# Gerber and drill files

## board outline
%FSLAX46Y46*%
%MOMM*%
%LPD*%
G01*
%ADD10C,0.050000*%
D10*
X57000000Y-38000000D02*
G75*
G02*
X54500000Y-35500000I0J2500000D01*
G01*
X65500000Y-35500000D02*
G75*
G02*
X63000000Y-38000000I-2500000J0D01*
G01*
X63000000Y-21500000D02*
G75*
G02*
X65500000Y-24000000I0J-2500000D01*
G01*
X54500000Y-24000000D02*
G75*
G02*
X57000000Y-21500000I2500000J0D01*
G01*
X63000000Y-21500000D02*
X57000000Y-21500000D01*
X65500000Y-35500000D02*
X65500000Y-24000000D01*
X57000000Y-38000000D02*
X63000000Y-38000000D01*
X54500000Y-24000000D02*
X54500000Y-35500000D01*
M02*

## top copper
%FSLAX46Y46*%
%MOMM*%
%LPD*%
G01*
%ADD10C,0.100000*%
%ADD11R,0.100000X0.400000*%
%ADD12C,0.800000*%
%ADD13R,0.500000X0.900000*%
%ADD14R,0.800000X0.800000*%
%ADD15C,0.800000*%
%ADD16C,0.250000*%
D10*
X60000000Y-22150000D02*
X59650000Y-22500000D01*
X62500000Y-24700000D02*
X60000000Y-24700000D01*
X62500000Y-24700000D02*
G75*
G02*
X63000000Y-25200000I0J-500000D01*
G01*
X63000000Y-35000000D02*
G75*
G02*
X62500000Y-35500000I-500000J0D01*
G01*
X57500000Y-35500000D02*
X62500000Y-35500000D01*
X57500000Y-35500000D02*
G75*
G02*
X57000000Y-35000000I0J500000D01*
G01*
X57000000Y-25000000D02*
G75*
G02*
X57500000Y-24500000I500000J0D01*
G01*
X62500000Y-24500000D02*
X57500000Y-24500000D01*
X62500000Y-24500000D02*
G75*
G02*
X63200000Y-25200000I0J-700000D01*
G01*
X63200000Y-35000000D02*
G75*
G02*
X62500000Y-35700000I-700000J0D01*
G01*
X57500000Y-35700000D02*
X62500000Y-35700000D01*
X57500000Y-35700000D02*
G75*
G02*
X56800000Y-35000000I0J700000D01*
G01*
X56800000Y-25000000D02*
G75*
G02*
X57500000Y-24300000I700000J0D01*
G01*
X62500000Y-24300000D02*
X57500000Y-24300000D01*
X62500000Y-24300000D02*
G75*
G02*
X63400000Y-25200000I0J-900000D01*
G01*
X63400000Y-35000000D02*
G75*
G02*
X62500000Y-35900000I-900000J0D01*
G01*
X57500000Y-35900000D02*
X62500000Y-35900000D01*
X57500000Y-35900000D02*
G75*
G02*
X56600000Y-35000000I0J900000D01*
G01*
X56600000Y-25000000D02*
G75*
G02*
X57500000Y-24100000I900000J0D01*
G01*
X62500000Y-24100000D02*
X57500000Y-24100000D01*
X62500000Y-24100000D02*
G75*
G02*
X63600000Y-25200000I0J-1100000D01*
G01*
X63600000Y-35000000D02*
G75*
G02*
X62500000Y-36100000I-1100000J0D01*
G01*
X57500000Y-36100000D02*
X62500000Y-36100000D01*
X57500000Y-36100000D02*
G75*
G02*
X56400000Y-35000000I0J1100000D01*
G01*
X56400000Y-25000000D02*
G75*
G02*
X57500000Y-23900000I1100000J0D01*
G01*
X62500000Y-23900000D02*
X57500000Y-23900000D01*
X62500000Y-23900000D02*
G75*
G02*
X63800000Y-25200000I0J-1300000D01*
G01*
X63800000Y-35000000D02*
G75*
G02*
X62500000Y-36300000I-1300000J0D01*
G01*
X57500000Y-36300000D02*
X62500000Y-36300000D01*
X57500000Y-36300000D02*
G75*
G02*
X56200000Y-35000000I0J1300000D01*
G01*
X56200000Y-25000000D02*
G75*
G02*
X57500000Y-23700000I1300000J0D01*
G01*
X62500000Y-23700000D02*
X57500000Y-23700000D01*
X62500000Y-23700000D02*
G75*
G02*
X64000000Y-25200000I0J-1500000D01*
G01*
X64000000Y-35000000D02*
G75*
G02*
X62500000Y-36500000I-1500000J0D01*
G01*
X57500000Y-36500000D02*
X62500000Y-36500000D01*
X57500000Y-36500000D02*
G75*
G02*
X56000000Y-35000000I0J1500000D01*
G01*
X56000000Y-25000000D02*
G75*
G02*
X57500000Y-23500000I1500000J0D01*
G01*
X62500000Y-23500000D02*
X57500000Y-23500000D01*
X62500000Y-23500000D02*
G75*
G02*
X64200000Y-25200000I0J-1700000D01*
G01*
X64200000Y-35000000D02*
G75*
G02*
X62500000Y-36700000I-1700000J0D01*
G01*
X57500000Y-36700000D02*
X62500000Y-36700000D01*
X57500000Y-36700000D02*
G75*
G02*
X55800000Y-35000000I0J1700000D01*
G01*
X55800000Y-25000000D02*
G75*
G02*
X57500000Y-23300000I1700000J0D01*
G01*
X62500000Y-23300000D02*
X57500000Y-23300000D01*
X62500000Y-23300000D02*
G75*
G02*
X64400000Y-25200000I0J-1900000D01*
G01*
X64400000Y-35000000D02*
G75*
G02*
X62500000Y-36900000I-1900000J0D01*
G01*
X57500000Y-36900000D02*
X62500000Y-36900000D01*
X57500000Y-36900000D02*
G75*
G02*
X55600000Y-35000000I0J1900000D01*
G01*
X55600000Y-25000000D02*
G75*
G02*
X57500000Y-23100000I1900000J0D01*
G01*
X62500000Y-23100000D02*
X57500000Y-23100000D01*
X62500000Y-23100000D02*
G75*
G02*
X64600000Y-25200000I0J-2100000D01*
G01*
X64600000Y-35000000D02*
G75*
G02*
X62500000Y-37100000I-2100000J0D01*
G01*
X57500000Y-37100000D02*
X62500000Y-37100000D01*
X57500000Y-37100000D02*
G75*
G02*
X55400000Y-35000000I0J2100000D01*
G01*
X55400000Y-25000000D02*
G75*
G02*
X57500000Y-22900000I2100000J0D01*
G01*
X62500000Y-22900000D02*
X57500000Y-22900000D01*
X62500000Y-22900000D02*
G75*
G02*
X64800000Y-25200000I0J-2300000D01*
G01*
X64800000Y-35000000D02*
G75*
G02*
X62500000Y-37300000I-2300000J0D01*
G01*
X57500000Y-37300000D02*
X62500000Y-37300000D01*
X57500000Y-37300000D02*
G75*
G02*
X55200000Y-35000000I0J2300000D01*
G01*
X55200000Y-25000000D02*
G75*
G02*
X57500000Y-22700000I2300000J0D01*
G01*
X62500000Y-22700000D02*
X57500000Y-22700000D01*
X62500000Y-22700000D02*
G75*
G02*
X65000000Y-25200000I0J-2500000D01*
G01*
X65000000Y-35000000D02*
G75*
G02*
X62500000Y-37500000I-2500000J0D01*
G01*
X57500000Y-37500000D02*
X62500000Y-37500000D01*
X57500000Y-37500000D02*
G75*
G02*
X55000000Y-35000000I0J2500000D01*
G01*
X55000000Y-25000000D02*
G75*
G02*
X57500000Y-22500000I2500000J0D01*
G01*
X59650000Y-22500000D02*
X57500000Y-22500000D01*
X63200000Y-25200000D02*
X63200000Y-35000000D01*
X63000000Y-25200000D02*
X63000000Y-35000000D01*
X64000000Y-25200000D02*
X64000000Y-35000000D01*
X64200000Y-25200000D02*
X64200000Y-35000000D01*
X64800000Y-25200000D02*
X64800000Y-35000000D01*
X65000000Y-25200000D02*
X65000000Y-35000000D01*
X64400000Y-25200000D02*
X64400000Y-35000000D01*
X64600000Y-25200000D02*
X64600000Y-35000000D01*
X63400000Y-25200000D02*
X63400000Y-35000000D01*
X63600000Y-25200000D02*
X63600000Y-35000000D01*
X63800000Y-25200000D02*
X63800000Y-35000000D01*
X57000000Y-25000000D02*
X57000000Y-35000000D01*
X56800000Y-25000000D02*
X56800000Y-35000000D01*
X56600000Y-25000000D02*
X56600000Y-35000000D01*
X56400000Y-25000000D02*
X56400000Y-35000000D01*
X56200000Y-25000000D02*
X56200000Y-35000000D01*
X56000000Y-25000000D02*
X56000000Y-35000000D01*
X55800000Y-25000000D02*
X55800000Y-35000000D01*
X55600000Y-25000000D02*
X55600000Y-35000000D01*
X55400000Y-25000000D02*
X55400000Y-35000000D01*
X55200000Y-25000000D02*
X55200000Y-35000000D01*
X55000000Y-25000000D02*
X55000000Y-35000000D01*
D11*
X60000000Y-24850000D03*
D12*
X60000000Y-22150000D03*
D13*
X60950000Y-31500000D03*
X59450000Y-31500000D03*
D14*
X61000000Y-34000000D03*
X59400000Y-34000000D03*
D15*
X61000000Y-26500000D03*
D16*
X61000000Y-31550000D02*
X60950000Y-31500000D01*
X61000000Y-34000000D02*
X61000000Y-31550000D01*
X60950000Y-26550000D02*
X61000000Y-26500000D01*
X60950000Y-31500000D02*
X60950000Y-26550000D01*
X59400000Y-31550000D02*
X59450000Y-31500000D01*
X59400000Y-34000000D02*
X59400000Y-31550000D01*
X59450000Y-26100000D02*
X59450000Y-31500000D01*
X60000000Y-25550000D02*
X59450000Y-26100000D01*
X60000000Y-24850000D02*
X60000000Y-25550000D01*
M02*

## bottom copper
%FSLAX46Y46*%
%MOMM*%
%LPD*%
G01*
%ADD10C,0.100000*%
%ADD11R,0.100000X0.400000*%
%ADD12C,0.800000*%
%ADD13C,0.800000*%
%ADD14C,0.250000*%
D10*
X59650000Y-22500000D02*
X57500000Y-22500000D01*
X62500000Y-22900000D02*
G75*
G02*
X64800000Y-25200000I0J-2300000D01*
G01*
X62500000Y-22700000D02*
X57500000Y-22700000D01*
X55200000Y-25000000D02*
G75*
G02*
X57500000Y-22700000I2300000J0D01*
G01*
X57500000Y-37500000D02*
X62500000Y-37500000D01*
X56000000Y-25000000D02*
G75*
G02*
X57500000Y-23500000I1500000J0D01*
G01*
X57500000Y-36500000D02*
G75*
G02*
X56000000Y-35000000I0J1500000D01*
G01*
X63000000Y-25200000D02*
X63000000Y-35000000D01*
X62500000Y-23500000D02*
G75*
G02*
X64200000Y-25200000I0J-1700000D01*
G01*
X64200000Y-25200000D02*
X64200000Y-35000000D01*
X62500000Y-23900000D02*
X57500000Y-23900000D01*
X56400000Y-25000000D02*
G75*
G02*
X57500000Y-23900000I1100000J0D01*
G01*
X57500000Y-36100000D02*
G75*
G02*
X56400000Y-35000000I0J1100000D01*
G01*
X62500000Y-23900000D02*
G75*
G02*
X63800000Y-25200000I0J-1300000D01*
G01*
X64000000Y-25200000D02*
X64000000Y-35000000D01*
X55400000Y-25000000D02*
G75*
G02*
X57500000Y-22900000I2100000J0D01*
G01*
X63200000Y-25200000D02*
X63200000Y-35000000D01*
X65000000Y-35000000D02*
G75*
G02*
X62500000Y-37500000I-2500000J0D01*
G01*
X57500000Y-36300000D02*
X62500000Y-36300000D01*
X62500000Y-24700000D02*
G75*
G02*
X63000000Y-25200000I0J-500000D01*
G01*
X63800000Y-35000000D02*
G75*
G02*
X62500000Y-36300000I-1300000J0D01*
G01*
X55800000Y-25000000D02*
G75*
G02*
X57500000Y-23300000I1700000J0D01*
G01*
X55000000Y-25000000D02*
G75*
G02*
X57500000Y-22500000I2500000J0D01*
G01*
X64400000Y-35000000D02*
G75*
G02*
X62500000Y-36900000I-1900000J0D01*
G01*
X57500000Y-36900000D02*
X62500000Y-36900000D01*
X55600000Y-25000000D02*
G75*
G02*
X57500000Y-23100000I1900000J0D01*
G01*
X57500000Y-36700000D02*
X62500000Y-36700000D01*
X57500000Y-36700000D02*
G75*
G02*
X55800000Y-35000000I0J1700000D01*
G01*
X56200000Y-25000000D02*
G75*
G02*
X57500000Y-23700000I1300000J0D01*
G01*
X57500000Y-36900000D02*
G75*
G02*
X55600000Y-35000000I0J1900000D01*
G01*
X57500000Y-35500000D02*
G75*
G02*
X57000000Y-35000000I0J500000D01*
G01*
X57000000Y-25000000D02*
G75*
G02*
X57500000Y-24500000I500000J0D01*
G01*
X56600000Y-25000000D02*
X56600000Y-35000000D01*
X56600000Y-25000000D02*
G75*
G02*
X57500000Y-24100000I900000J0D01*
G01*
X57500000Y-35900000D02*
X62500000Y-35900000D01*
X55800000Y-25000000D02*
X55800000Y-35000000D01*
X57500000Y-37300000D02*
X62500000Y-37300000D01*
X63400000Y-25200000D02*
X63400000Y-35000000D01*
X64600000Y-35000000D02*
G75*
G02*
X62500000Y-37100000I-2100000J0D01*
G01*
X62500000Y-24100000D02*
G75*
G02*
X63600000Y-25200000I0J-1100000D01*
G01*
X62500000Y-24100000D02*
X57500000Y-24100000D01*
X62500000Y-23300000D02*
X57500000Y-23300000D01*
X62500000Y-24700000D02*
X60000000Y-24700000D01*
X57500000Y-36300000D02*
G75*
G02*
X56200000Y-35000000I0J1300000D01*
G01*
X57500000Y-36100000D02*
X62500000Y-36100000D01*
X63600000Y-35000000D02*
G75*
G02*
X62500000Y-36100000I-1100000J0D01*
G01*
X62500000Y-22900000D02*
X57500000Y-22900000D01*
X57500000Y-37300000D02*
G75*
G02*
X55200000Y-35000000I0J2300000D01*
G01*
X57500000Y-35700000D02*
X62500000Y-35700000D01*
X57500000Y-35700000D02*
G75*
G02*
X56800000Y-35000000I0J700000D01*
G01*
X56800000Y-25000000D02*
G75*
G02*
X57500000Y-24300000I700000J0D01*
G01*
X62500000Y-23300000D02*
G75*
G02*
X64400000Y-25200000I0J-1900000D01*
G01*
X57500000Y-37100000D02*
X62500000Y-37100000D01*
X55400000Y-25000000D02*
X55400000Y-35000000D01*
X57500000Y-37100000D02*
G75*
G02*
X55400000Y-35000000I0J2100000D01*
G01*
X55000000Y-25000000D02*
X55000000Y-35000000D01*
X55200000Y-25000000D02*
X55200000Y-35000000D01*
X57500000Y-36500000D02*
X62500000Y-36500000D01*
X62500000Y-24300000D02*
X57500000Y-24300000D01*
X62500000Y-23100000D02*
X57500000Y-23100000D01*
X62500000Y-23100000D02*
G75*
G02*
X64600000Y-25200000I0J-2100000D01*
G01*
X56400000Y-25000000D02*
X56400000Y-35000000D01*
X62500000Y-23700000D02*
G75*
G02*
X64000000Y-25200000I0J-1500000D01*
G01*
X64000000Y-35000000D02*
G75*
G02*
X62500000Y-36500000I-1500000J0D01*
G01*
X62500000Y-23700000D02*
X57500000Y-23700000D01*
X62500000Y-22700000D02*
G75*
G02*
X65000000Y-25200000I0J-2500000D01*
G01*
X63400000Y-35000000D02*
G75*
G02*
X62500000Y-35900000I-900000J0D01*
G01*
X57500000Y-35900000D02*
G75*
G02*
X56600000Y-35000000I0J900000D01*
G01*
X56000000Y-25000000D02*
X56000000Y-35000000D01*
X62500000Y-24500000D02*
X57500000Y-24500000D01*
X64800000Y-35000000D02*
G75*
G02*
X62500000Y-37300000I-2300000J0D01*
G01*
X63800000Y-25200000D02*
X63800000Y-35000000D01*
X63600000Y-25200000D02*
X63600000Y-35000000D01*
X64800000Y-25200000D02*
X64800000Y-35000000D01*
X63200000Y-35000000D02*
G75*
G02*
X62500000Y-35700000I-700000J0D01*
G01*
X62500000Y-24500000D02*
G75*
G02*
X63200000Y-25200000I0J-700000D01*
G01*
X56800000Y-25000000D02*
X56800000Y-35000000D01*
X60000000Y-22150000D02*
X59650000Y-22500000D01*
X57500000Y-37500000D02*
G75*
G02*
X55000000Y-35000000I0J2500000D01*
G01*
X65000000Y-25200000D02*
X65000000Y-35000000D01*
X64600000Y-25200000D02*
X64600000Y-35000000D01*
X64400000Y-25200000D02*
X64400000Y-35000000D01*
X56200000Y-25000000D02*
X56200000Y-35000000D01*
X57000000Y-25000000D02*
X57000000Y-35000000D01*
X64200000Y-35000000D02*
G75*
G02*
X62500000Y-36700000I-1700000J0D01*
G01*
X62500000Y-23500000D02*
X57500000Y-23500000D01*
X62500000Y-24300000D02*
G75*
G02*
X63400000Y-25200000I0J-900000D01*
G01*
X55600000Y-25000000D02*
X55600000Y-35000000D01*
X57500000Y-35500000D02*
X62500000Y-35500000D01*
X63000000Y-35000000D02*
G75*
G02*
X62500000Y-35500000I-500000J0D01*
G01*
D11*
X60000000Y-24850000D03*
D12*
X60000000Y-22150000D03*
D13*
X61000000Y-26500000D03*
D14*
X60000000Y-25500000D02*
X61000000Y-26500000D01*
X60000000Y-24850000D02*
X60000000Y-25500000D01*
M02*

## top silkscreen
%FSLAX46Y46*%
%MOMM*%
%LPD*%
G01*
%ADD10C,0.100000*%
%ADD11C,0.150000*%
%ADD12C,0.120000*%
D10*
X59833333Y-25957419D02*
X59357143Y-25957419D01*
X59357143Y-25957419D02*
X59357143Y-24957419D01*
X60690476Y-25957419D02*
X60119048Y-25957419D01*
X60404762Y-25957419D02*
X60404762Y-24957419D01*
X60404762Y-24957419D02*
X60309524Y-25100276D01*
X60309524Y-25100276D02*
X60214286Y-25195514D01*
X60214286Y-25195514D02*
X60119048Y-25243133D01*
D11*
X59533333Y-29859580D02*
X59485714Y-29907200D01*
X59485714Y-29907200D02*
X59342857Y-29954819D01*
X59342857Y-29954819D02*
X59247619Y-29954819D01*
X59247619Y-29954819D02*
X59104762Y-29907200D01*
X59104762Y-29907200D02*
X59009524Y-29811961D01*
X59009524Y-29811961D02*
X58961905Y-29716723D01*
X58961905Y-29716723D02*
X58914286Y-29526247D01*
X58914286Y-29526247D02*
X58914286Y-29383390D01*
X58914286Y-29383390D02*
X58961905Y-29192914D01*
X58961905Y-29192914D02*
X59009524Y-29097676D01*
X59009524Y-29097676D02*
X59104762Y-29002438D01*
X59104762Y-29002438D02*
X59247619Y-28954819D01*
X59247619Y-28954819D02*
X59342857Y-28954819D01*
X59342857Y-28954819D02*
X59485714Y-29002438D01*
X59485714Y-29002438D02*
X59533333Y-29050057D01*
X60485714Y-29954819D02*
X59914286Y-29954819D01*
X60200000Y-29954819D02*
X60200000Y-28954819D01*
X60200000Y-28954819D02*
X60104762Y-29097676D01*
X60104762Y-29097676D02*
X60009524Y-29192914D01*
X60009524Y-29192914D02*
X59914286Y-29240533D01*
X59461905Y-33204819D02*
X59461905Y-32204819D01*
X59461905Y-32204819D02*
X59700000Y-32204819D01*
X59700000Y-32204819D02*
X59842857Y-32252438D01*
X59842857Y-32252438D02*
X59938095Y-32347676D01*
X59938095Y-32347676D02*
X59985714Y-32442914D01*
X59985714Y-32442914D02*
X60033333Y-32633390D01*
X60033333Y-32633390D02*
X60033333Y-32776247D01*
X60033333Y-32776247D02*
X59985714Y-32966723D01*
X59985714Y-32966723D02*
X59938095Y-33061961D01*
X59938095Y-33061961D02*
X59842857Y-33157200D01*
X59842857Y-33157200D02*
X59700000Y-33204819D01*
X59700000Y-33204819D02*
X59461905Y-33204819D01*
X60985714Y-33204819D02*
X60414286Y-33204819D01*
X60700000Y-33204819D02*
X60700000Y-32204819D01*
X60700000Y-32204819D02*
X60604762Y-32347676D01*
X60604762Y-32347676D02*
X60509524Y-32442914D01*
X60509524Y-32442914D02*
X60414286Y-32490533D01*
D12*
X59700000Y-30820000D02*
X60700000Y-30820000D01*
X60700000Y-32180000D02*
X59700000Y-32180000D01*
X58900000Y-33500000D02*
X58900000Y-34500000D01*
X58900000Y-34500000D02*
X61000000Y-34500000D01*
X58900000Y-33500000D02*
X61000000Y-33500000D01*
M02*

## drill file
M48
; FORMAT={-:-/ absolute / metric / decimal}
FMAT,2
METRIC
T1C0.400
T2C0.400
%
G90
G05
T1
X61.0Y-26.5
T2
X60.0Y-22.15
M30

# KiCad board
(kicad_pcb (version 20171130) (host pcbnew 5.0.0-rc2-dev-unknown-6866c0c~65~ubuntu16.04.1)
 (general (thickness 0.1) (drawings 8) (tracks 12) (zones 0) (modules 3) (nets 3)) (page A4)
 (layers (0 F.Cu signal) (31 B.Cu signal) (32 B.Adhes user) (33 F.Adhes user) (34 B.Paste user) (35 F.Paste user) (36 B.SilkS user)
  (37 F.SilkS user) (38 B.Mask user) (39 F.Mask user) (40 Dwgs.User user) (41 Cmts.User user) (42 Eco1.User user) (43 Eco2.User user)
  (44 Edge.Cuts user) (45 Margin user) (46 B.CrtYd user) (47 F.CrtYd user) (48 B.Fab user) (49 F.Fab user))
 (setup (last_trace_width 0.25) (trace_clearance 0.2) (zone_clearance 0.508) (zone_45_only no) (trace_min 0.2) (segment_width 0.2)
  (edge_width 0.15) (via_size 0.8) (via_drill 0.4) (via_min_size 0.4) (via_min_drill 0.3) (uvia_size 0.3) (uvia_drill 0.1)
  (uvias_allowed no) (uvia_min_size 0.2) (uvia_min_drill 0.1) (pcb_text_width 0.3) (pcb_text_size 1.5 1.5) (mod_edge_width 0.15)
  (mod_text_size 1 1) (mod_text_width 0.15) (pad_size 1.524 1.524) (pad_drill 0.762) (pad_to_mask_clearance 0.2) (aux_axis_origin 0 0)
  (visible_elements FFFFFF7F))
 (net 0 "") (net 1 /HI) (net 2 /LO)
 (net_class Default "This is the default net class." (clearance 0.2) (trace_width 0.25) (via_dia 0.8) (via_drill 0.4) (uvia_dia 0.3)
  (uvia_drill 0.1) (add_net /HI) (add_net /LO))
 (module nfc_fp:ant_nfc (layer F.Cu) (at 60 30)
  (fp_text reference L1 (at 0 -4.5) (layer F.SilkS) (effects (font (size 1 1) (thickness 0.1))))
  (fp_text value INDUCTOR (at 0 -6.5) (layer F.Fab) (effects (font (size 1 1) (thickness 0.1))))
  (fp_line (start -0.35 -7.5) (end -2.5 -7.5) (layer B.Cu) (width 0.1))
  (fp_arc (start 2.5 -4.8) (end 4.8 -4.8) (angle -90) (layer B.Cu) (width 0.1))
  (fp_line (start 2.5 -7.3) (end -2.5 -7.3) (layer B.Cu) (width 0.1))
  (fp_arc (start -2.5 -5) (end -2.5 -7.3) (angle -90) (layer B.Cu) (width 0.1))
  (fp_line (start -2.5 7.5) (end 2.5 7.5) (layer B.Cu) (width 0.1))
  (fp_arc (start -2.5 -5) (end -2.5 -6.5) (angle -90) (layer B.Cu) (width 0.1))
  (fp_arc (start -2.5 5) (end -4 5) (angle -90) (layer B.Cu) (width 0.1)) (fp_line (start 3 -4.8) (end 3 5) (layer B.Cu) (width 0.1))
  (fp_arc (start 2.5 -4.8) (end 4.2 -4.8) (angle -90) (layer B.Cu) (width 0.1))
  (fp_line (start 4.2 -4.8) (end 4.2 5) (layer B.Cu) (width 0.1))
  (fp_line (start 2.5 -6.1) (end -2.5 -6.1) (layer B.Cu) (width 0.1))
  (fp_arc (start -2.5 -5) (end -2.5 -6.1) (angle -90) (layer B.Cu) (width 0.1))
  (fp_arc (start -2.5 5) (end -3.6 5) (angle -90) (layer B.Cu) (width 0.1))
  (fp_arc (start 2.5 -4.8) (end 3.8 -4.8) (angle -90) (layer B.Cu) (width 0.1)) (fp_line (start 4 -4.8) (end 4 5) (layer B.Cu) (width 0.1))
  (fp_arc (start -2.5 -5) (end -2.5 -7.1) (angle -90) (layer B.Cu) (width 0.1))
  (fp_line (start 3.2 -4.8) (end 3.2 5) (layer B.Cu) (width 0.1))
  (fp_arc (start 2.5 5) (end 2.5 7.5) (angle -90) (layer B.Cu) (width 0.1))
  (fp_line (start -2.5 6.3) (end 2.5 6.3) (layer B.Cu) (width 0.1))
  (fp_arc (start 2.5 -4.8) (end 3 -4.8) (angle -90) (layer B.Cu) (width 0.1))
  (fp_arc (start 2.5 5) (end 2.5 6.3) (angle -90) (layer B.Cu) (width 0.1))
  (fp_arc (start -2.5 -5) (end -2.5 -6.7) (angle -90) (layer B.Cu) (width 0.1))
  (fp_arc (start -2.5 -5) (end -2.5 -7.5) (angle -90) (layer B.Cu) (width 0.1))
  (fp_arc (start 2.5 5) (end 2.5 6.9) (angle -90) (layer B.Cu) (width 0.1))
  (fp_line (start -2.5 6.9) (end 2.5 6.9) (layer B.Cu) (width 0.1))
  (fp_arc (start -2.5 -5) (end -2.5 -6.9) (angle -90) (layer B.Cu) (width 0.1))
  (fp_line (start -2.5 6.7) (end 2.5 6.7) (layer B.Cu) (width 0.1))
  (fp_arc (start -2.5 5) (end -4.2 5) (angle -90) (layer B.Cu) (width 0.1))
  (fp_arc (start -2.5 -5) (end -2.5 -6.3) (angle -90) (layer B.Cu) (width 0.1))
  (fp_arc (start -2.5 5) (end -4.4 5) (angle -90) (layer B.Cu) (width 0.1))
  (fp_arc (start -2.5 5) (end -3 5) (angle -90) (layer B.Cu) (width 0.1))
  (fp_arc (start -2.5 -5) (end -2.5 -5.5) (angle -90) (layer B.Cu) (width 0.1))
  (fp_line (start -3.4 -5) (end -3.4 5) (layer B.Cu) (width 0.1))
  (fp_arc (start -2.5 -5) (end -2.5 -5.9) (angle -90) (layer B.Cu) (width 0.1))
  (fp_line (start -2.5 5.9) (end 2.5 5.9) (layer B.Cu) (width 0.1))
  (fp_line (start -4.2 -5) (end -4.2 5) (layer B.Cu) (width 0.1))
  (fp_line (start -2.5 7.3) (end 2.5 7.3) (layer B.Cu) (width 0.1))
  (fp_line (start 3.4 -4.8) (end 3.4 5) (layer B.Cu) (width 0.1))
  (fp_arc (start 2.5 5) (end 2.5 7.1) (angle -90) (layer B.Cu) (width 0.1))
  (fp_arc (start 2.5 -4.8) (end 3.6 -4.8) (angle -90) (layer B.Cu) (width 0.1))
  (fp_line (start 2.5 -5.9) (end -2.5 -5.9) (layer B.Cu) (width 0.1))
  (fp_line (start 2.5 -6.7) (end -2.5 -6.7) (layer B.Cu) (width 0.1))
  (fp_line (start 2.5 -5.3) (end 0 -5.3) (layer B.Cu) (width 0.1))
  (fp_arc (start -2.5 5) (end -3.8 5) (angle -90) (layer B.Cu) (width 0.1))
  (fp_line (start -2.5 6.1) (end 2.5 6.1) (layer B.Cu) (width 0.1))
  (fp_arc (start 2.5 5) (end 2.5 6.1) (angle -90) (layer B.Cu) (width 0.1))
  (fp_line (start 2.5 -7.1) (end -2.5 -7.1) (layer B.Cu) (width 0.1))
  (fp_arc (start -2.5 5) (end -4.8 5) (angle -90) (layer B.Cu) (width 0.1))
  (fp_line (start -2.5 5.7) (end 2.5 5.7) (layer B.Cu) (width 0.1))
  (fp_arc (start -2.5 5) (end -3.2 5) (angle -90) (layer B.Cu) (width 0.1))
  (fp_arc (start -2.5 -5) (end -2.5 -5.7) (angle -90) (layer B.Cu) (width 0.1))
  (fp_arc (start 2.5 -4.8) (end 4.4 -4.8) (angle -90) (layer B.Cu) (width 0.1))
  (fp_line (start -2.5 7.1) (end 2.5 7.1) (layer B.Cu) (width 0.1))
  (fp_line (start -4.6 -5) (end -4.6 5) (layer B.Cu) (width 0.1))
  (fp_arc (start -2.5 5) (end -4.6 5) (angle -90) (layer B.Cu) (width 0.1)) (fp_line (start -5 -5) (end -5 5) (layer B.Cu) (width 0.1))
  (fp_line (start -4.8 -5) (end -4.8 5) (layer B.Cu) (width 0.1))
  (fp_line (start -2.5 6.5) (end 2.5 6.5) (layer B.Cu) (width 0.1))
  (fp_line (start 2.5 -5.7) (end -2.5 -5.7) (layer B.Cu) (width 0.1))
  (fp_line (start 2.5 -6.9) (end -2.5 -6.9) (layer B.Cu) (width 0.1))
  (fp_arc (start 2.5 -4.8) (end 4.6 -4.8) (angle -90) (layer B.Cu) (width 0.1))
  (fp_line (start -3.6 -5) (end -3.6 5) (layer B.Cu) (width 0.1))
  (fp_arc (start 2.5 -4.8) (end 4 -4.8) (angle -90) (layer B.Cu) (width 0.1))
  (fp_arc (start 2.5 5) (end 2.5 6.5) (angle -90) (layer B.Cu) (width 0.1))
  (fp_line (start 2.5 -6.3) (end -2.5 -6.3) (layer B.Cu) (width 0.1))
  (fp_arc (start 2.5 -4.8) (end 5 -4.8) (angle -90) (layer B.Cu) (width 0.1))
  (fp_arc (start 2.5 5) (end 2.5 5.9) (angle -90) (layer B.Cu) (width 0.1))
  (fp_arc (start -2.5 5) (end -3.4 5) (angle -90) (layer B.Cu) (width 0.1)) (fp_line (start -4 -5) (end -4 5) (layer B.Cu) (width 0.1))
  (fp_line (start 2.5 -5.5) (end -2.5 -5.5) (layer B.Cu) (width 0.1))
  (fp_arc (start 2.5 5) (end 2.5 7.3) (angle -90) (layer B.Cu) (width 0.1))
  (fp_line (start 3.8 -4.8) (end 3.8 5) (layer B.Cu) (width 0.1))
  (fp_line (start 3.6 -4.8) (end 3.6 5) (layer B.Cu) (width 0.1))
  (fp_line (start 4.8 -4.8) (end 4.8 5) (layer B.Cu) (width 0.1))
  (fp_arc (start 2.5 5) (end 2.5 5.7) (angle -90) (layer B.Cu) (width 0.1))
  (fp_arc (start 2.5 -4.8) (end 3.2 -4.8) (angle -90) (layer B.Cu) (width 0.1))
  (fp_line (start -3.2 -5) (end -3.2 5) (layer B.Cu) (width 0.1))
  (fp_line (start 0 -7.85) (end -0.35 -7.5) (layer B.Cu) (width 0.1))
  (fp_arc (start -2.5 5) (end -5 5) (angle -90) (layer B.Cu) (width 0.1)) (fp_line (start 5 -4.8) (end 5 5) (layer B.Cu) (width 0.1))
  (fp_line (start 4.6 -4.8) (end 4.6 5) (layer B.Cu) (width 0.1))
  (fp_line (start 4.4 -4.8) (end 4.4 5) (layer B.Cu) (width 0.1))
  (fp_line (start -3.8 -5) (end -3.8 5) (layer B.Cu) (width 0.1)) (fp_line (start -3 -5) (end -3 5) (layer B.Cu) (width 0.1))
  (fp_arc (start 2.5 5) (end 2.5 6.7) (angle -90) (layer B.Cu) (width 0.1))
  (fp_line (start 2.5 -6.5) (end -2.5 -6.5) (layer B.Cu) (width 0.1))
  (fp_arc (start 2.5 -4.8) (end 3.4 -4.8) (angle -90) (layer B.Cu) (width 0.1))
  (fp_line (start -4.4 -5) (end -4.4 5) (layer B.Cu) (width 0.1))
  (fp_line (start -2.5 5.5) (end 2.5 5.5) (layer B.Cu) (width 0.1))
  (fp_arc (start 2.5 5) (end 2.5 5.5) (angle -90) (layer B.Cu) (width 0.1))
  (fp_line (start 0 -7.85) (end -0.35 -7.5) (layer F.Cu) (width 0.1))
  (fp_line (start 2.5 -5.3) (end 0 -5.3) (layer F.Cu) (width 0.1))
  (fp_arc (start 2.5 -4.8) (end 3 -4.8) (angle -90) (layer F.Cu) (width 0.1))
  (fp_arc (start 2.5 5) (end 2.5 5.5) (angle -90) (layer F.Cu) (width 0.1))
  (fp_line (start -2.5 5.5) (end 2.5 5.5) (layer F.Cu) (width 0.1))
  (fp_arc (start -2.5 5) (end -3 5) (angle -90) (layer F.Cu) (width 0.1))
  (fp_arc (start -2.5 -5) (end -2.5 -5.5) (angle -90) (layer F.Cu) (width 0.1))
  (fp_line (start 2.5 -5.5) (end -2.5 -5.5) (layer F.Cu) (width 0.1))
  (fp_arc (start 2.5 -4.8) (end 3.2 -4.8) (angle -90) (layer F.Cu) (width 0.1))
  (fp_arc (start 2.5 5) (end 2.5 5.7) (angle -90) (layer F.Cu) (width 0.1))
  (fp_line (start -2.5 5.7) (end 2.5 5.7) (layer F.Cu) (width 0.1))
  (fp_arc (start -2.5 5) (end -3.2 5) (angle -90) (layer F.Cu) (width 0.1))
  (fp_arc (start -2.5 -5) (end -2.5 -5.7) (angle -90) (layer F.Cu) (width 0.1))
  (fp_line (start 2.5 -5.7) (end -2.5 -5.7) (layer F.Cu) (width 0.1))
  (fp_arc (start 2.5 -4.8) (end 3.4 -4.8) (angle -90) (layer F.Cu) (width 0.1))
  (fp_arc (start 2.5 5) (end 2.5 5.9) (angle -90) (layer F.Cu) (width 0.1))
  (fp_line (start -2.5 5.9) (end 2.5 5.9) (layer F.Cu) (width 0.1))
  (fp_arc (start -2.5 5) (end -3.4 5) (angle -90) (layer F.Cu) (width 0.1))
  (fp_arc (start -2.5 -5) (end -2.5 -5.9) (angle -90) (layer F.Cu) (width 0.1))
  (fp_line (start 2.5 -5.9) (end -2.5 -5.9) (layer F.Cu) (width 0.1))
  (fp_arc (start 2.5 -4.8) (end 3.6 -4.8) (angle -90) (layer F.Cu) (width 0.1))
  (fp_arc (start 2.5 5) (end 2.5 6.1) (angle -90) (layer F.Cu) (width 0.1))
  (fp_line (start -2.5 6.1) (end 2.5 6.1) (layer F.Cu) (width 0.1))
  (fp_arc (start -2.5 5) (end -3.6 5) (angle -90) (layer F.Cu) (width 0.1))
  (fp_arc (start -2.5 -5) (end -2.5 -6.1) (angle -90) (layer F.Cu) (width 0.1))
  (fp_line (start 2.5 -6.1) (end -2.5 -6.1) (layer F.Cu) (width 0.1))
  (fp_arc (start 2.5 -4.8) (end 3.8 -4.8) (angle -90) (layer F.Cu) (width 0.1))
  (fp_arc (start 2.5 5) (end 2.5 6.3) (angle -90) (layer F.Cu) (width 0.1))
  (fp_line (start -2.5 6.3) (end 2.5 6.3) (layer F.Cu) (width 0.1))
  (fp_arc (start -2.5 5) (end -3.8 5) (angle -90) (layer F.Cu) (width 0.1))
  (fp_arc (start -2.5 -5) (end -2.5 -6.3) (angle -90) (layer F.Cu) (width 0.1))
  (fp_line (start 2.5 -6.3) (end -2.5 -6.3) (layer F.Cu) (width 0.1))
  (fp_arc (start 2.5 -4.8) (end 4 -4.8) (angle -90) (layer F.Cu) (width 0.1))
  (fp_arc (start 2.5 5) (end 2.5 6.5) (angle -90) (layer F.Cu) (width 0.1))
  (fp_line (start -2.5 6.5) (end 2.5 6.5) (layer F.Cu) (width 0.1))
  (fp_arc (start -2.5 5) (end -4 5) (angle -90) (layer F.Cu) (width 0.1))
  (fp_arc (start -2.5 -5) (end -2.5 -6.5) (angle -90) (layer F.Cu) (width 0.1))
  (fp_line (start 2.5 -6.5) (end -2.5 -6.5) (layer F.Cu) (width 0.1))
  (fp_arc (start 2.5 -4.8) (end 4.2 -4.8) (angle -90) (layer F.Cu) (width 0.1))
  (fp_arc (start 2.5 5) (end 2.5 6.7) (angle -90) (layer F.Cu) (width 0.1))
  (fp_line (start -2.5 6.7) (end 2.5 6.7) (layer F.Cu) (width 0.1))
  (fp_arc (start -2.5 5) (end -4.2 5) (angle -90) (layer F.Cu) (width 0.1))
  (fp_arc (start -2.5 -5) (end -2.5 -6.7) (angle -90) (layer F.Cu) (width 0.1))
  (fp_line (start 2.5 -6.7) (end -2.5 -6.7) (layer F.Cu) (width 0.1))
  (fp_arc (start 2.5 -4.8) (end 4.4 -4.8) (angle -90) (layer F.Cu) (width 0.1))
  (fp_arc (start 2.5 5) (end 2.5 6.9) (angle -90) (layer F.Cu) (width 0.1))
  (fp_line (start -2.5 6.9) (end 2.5 6.9) (layer F.Cu) (width 0.1))
  (fp_arc (start -2.5 5) (end -4.4 5) (angle -90) (layer F.Cu) (width 0.1))
  (fp_arc (start -2.5 -5) (end -2.5 -6.9) (angle -90) (layer F.Cu) (width 0.1))
  (fp_line (start 2.5 -6.9) (end -2.5 -6.9) (layer F.Cu) (width 0.1))
  (fp_arc (start 2.5 -4.8) (end 4.6 -4.8) (angle -90) (layer F.Cu) (width 0.1))
  (fp_arc (start 2.5 5) (end 2.5 7.1) (angle -90) (layer F.Cu) (width 0.1))
  (fp_line (start -2.5 7.1) (end 2.5 7.1) (layer F.Cu) (width 0.1))
  (fp_arc (start -2.5 5) (end -4.6 5) (angle -90) (layer F.Cu) (width 0.1))
  (fp_arc (start -2.5 -5) (end -2.5 -7.1) (angle -90) (layer F.Cu) (width 0.1))
  (fp_line (start 2.5 -7.1) (end -2.5 -7.1) (layer F.Cu) (width 0.1))
  (fp_arc (start 2.5 -4.8) (end 4.8 -4.8) (angle -90) (layer F.Cu) (width 0.1))
  (fp_arc (start 2.5 5) (end 2.5 7.3) (angle -90) (layer F.Cu) (width 0.1))
  (fp_line (start -2.5 7.3) (end 2.5 7.3) (layer F.Cu) (width 0.1))
  (fp_arc (start -2.5 5) (end -4.8 5) (angle -90) (layer F.Cu) (width 0.1))
  (fp_arc (start -2.5 -5) (end -2.5 -7.3) (angle -90) (layer F.Cu) (width 0.1))
  (fp_line (start 2.5 -7.3) (end -2.5 -7.3) (layer F.Cu) (width 0.1))
  (fp_arc (start 2.5 -4.8) (end 5 -4.8) (angle -90) (layer F.Cu) (width 0.1))
  (fp_arc (start 2.5 5) (end 2.5 7.5) (angle -90) (layer F.Cu) (width 0.1))
  (fp_line (start -2.5 7.5) (end 2.5 7.5) (layer F.Cu) (width 0.1))
  (fp_arc (start -2.5 5) (end -5 5) (angle -90) (layer F.Cu) (width 0.1))
  (fp_arc (start -2.5 -5) (end -2.5 -7.5) (angle -90) (layer F.Cu) (width 0.1))
  (fp_line (start -0.35 -7.5) (end -2.5 -7.5) (layer F.Cu) (width 0.1))
  (fp_line (start 3.2 -4.8) (end 3.2 5) (layer F.Cu) (width 0.1)) (fp_line (start 3 -4.8) (end 3 5) (layer F.Cu) (width 0.1))
  (fp_line (start 4 -4.8) (end 4 5) (layer F.Cu) (width 0.1))
  (fp_line (start 4.2 -4.8) (end 4.2 5) (layer F.Cu) (width 0.1))
  (fp_line (start 4.8 -4.8) (end 4.8 5) (layer F.Cu) (width 0.1)) (fp_line (start 5 -4.8) (end 5 5) (layer F.Cu) (width 0.1))
  (fp_line (start 4.4 -4.8) (end 4.4 5) (layer F.Cu) (width 0.1))
  (fp_line (start 4.6 -4.8) (end 4.6 5) (layer F.Cu) (width 0.1))
  (fp_line (start 3.4 -4.8) (end 3.4 5) (layer F.Cu) (width 0.1))
  (fp_line (start 3.6 -4.8) (end 3.6 5) (layer F.Cu) (width 0.1))
  (fp_line (start 3.8 -4.8) (end 3.8 5) (layer F.Cu) (width 0.1)) (fp_line (start -3 -5) (end -3 5) (layer F.Cu) (width 0.1))
  (fp_line (start -3.2 -5) (end -3.2 5) (layer F.Cu) (width 0.1))
  (fp_line (start -3.4 -5) (end -3.4 5) (layer F.Cu) (width 0.1))
  (fp_line (start -3.6 -5) (end -3.6 5) (layer F.Cu) (width 0.1))
  (fp_line (start -3.8 -5) (end -3.8 5) (layer F.Cu) (width 0.1)) (fp_line (start -4 -5) (end -4 5) (layer F.Cu) (width 0.1))
  (fp_line (start -4.2 -5) (end -4.2 5) (layer F.Cu) (width 0.1))
  (fp_line (start -4.4 -5) (end -4.4 5) (layer F.Cu) (width 0.1))
  (fp_line (start -4.6 -5) (end -4.6 5) (layer F.Cu) (width 0.1))
  (fp_line (start -4.8 -5) (end -4.8 5) (layer F.Cu) (width 0.1)) (fp_line (start -5 -5) (end -5 5) (layer F.Cu) (width 0.1))
  (pad 2 smd rect (at 0 -5.15) (size 0.1 0.4) (layers B.Cu F.Paste F.Mask) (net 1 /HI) (clearance 0.04))
  (pad 1 smd rect (at 0 -5.15) (size 0.1 0.4) (layers F.Cu F.Paste F.Mask) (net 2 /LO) (clearance 0.04))
  (pad 3 thru_hole circle (at 0 -7.85 180) (size 0.8 0.8) (drill 0.4) (layers *.Cu *.Mask) (clearance 0.05)))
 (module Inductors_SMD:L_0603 (layer F.Cu) (at 60.2 31.5 180)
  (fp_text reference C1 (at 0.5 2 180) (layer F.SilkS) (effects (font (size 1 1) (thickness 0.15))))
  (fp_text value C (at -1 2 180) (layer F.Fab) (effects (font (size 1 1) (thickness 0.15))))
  (fp_line (start 0.5 0.68) (end -0.5 0.68) (layer F.SilkS) (width 0.12))
  (fp_line (start -0.5 -0.68) (end 0.5 -0.68) (layer F.SilkS) (width 0.12))
  (pad 1 smd rect (at -0.75 0 180) (size 0.5 0.9) (layers F.Cu F.Paste F.Mask) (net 1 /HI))
  (pad 2 smd rect (at 0.75 0 180) (size 0.5 0.9) (layers F.Cu F.Paste F.Mask) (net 2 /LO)))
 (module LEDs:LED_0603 (layer F.Cu) (at 60.2 34)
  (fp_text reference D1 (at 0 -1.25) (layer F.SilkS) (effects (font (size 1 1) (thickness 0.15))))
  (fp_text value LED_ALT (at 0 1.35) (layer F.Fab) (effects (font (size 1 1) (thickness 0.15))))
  (fp_line (start -1.3 -0.5) (end -1.3 0.5) (layer F.SilkS) (width 0.12))
  (fp_line (start -1.3 0.5) (end 0.8 0.5) (layer F.SilkS) (width 0.12))
  (fp_line (start -1.3 -0.5) (end 0.8 -0.5) (layer F.SilkS) (width 0.12))
  (pad 2 smd rect (at 0.8 0 180) (size 0.8 0.8) (layers F.Cu F.Paste F.Mask) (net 1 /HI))
  (pad 1 smd rect (at -0.8 0 180) (size 0.8 0.8) (layers F.Cu F.Paste F.Mask) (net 2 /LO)))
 (gr_arc (start 57 35.5) (end 54.5 35.5) (angle -90) (layer Edge.Cuts) (width 0.05))
 (gr_arc (start 63 35.5) (end 63 38) (angle -90) (layer Edge.Cuts) (width 0.05))
 (gr_arc (start 63 24) (end 65.5 24) (angle -90) (layer Edge.Cuts) (width 0.05))
 (gr_arc (start 57 24) (end 57 21.5) (angle -90) (layer Edge.Cuts) (width 0.05))
 (gr_line (start 63 21.5) (end 57 21.5) (layer Edge.Cuts) (width 0.05))
 (gr_line (start 65.5 35.5) (end 65.5 24) (layer Edge.Cuts) (width 0.05))
 (gr_line (start 57 38) (end 63 38) (layer Edge.Cuts) (width 0.05))
 (gr_line (start 54.5 24) (end 54.5 35.5) (layer Edge.Cuts) (width 0.05))
 (segment (start 61 31.55) (end 60.95 31.5) (width 0.25) (layer F.Cu) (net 1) (status 30))
 (segment (start 61 34) (end 61 31.55) (width 0.25) (layer F.Cu) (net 1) (status 30))
 (via (at 61 26.5) (size 0.8) (drill 0.4) (layers F.Cu B.Cu) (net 1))
 (segment (start 60.95 26.55) (end 61 26.5) (width 0.25) (layer F.Cu) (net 1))
 (segment (start 60.95 31.5) (end 60.95 26.55) (width 0.25) (layer F.Cu) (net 1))
 (segment (start 60 25.5) (end 61 26.5) (width 0.25) (layer B.Cu) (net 1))
 (segment (start 60 24.85) (end 60 25.5) (width 0.25) (layer B.Cu) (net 1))
 (segment (start 59.4 31.55) (end 59.45 31.5) (width 0.25) (layer F.Cu) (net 2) (status 30))
 (segment (start 59.4 34) (end 59.4 31.55) (width 0.25) (layer F.Cu) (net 2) (status 30))
 (segment (start 59.45 26.1) (end 59.45 31.5) (width 0.25) (layer F.Cu) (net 2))
 (segment (start 60 25.55) (end 59.45 26.1) (width 0.25) (layer F.Cu) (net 2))
 (segment (start 60 24.85) (end 60 25.55) (width 0.25) (layer F.Cu) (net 2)))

